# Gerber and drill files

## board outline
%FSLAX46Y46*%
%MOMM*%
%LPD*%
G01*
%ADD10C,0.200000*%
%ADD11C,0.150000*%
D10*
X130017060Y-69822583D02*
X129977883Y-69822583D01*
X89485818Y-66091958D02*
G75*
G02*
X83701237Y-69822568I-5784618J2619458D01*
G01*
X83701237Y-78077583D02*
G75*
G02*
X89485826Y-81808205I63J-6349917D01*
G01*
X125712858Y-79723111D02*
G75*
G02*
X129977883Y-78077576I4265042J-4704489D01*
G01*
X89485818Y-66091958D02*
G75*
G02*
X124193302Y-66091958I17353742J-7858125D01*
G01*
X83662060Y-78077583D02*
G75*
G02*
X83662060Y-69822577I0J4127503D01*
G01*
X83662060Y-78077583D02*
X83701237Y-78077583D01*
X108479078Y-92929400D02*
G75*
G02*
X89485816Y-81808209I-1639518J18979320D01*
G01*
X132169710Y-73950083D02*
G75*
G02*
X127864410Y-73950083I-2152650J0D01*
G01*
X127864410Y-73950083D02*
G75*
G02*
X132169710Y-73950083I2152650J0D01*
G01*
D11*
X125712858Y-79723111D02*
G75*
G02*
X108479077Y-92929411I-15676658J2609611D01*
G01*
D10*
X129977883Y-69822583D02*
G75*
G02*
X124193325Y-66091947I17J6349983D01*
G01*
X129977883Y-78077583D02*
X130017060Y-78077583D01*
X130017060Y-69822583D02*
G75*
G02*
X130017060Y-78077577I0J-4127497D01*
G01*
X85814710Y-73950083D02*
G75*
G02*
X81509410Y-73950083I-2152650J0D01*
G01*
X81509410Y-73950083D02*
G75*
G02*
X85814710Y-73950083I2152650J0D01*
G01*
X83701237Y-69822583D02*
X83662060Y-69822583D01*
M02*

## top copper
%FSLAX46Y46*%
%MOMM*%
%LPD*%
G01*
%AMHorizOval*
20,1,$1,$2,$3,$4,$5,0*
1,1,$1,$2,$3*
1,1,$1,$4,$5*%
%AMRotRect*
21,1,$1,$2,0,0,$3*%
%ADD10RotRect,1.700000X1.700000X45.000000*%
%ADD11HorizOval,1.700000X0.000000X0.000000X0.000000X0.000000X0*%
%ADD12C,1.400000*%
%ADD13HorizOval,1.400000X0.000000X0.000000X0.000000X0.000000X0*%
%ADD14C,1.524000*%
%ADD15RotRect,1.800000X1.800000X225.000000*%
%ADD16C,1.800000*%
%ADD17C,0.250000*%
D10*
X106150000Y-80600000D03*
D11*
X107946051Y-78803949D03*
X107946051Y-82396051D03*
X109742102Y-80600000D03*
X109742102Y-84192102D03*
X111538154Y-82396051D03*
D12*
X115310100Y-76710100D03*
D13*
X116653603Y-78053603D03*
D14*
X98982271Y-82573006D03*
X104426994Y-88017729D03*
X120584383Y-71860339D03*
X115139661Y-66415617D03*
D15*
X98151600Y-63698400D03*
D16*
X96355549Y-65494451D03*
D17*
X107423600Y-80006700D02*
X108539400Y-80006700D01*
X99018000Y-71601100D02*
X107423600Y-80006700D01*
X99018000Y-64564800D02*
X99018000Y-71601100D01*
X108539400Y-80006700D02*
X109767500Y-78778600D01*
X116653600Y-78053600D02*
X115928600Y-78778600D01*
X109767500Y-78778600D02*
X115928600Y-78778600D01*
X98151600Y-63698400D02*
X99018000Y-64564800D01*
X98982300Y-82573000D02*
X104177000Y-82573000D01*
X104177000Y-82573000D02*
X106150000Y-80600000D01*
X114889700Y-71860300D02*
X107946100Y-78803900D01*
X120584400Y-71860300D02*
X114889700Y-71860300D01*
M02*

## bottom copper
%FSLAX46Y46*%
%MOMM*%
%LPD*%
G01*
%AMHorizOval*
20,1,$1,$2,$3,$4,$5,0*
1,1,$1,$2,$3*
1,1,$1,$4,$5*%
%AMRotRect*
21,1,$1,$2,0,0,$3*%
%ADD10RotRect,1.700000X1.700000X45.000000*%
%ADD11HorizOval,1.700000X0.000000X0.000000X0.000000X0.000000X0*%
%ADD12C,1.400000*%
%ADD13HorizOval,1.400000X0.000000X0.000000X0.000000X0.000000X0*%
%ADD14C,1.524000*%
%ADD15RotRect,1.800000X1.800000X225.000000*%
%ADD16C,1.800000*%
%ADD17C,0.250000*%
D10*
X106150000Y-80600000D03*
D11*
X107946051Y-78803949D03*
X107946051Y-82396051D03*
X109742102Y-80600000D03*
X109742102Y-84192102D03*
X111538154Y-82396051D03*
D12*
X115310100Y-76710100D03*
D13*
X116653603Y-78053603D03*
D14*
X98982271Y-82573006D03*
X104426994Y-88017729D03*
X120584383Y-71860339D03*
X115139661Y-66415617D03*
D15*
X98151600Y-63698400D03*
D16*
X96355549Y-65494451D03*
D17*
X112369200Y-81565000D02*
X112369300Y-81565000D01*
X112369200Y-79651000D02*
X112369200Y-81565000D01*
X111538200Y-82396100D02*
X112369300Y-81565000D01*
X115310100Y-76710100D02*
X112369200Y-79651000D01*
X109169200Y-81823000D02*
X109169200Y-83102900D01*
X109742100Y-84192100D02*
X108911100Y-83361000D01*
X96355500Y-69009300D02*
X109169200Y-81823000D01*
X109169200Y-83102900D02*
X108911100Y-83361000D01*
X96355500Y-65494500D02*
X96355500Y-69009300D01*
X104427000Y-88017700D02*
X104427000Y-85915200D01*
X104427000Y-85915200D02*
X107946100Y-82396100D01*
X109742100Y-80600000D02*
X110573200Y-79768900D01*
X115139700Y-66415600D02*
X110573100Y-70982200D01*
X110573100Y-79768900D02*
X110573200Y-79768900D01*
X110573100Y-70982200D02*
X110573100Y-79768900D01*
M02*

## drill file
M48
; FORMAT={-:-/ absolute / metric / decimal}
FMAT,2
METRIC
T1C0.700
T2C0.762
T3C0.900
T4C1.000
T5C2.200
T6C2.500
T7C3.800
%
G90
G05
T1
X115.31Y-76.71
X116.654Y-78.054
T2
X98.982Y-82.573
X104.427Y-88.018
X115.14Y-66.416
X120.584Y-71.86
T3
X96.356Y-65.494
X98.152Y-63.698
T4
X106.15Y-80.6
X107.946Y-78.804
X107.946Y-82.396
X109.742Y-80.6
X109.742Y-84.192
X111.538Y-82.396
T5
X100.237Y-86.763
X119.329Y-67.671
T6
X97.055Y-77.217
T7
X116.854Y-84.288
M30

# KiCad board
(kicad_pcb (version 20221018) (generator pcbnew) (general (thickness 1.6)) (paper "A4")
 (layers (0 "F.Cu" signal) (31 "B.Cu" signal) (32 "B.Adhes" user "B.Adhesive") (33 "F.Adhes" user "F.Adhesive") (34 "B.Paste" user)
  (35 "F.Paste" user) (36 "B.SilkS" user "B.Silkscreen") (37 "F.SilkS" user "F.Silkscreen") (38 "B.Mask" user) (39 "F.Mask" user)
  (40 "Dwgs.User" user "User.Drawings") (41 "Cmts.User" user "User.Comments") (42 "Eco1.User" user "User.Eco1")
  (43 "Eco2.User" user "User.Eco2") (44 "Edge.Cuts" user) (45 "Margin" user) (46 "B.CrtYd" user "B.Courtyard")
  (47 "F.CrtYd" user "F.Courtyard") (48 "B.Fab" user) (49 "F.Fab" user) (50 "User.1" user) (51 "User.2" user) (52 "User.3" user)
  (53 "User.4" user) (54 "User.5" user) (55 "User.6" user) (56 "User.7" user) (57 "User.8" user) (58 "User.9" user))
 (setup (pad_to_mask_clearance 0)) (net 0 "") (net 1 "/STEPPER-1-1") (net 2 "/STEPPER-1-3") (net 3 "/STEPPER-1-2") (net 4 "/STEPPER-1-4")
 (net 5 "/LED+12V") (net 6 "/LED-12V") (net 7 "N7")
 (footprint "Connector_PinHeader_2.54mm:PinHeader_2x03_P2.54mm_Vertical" (layer "F.Cu") (at 106.15 80.6 45)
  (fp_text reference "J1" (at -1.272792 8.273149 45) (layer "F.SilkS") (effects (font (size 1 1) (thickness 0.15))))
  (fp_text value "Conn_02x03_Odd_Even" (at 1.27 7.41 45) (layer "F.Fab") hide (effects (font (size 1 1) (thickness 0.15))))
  (pad "1" thru_hole rect (at 0 0 45) (size 1.7 1.7) (drill 1) (layers "*.Cu" "*.Mask") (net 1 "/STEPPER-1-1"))
  (pad "2" thru_hole oval (at 2.54 0 45) (size 1.7 1.7) (drill 1) (layers "*.Cu" "*.Mask") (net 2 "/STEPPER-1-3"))
  (pad "3" thru_hole oval (at 0 2.54 45) (size 1.7 1.7) (drill 1) (layers "*.Cu" "*.Mask") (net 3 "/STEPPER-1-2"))
  (pad "4" thru_hole oval (at 2.54 2.54 45) (size 1.7 1.7) (drill 1) (layers "*.Cu" "*.Mask") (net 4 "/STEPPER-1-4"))
  (pad "5" thru_hole oval (at 0 5.08 45) (size 1.7 1.7) (drill 1) (layers "*.Cu" "*.Mask") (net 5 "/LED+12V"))
  (pad "6" thru_hole oval (at 2.54 5.08 45) (size 1.7 1.7) (drill 1) (layers "*.Cu" "*.Mask") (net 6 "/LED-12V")))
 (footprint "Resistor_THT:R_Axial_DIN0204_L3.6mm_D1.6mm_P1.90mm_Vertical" (layer "F.Cu") (at 115.3101 76.7101 -45)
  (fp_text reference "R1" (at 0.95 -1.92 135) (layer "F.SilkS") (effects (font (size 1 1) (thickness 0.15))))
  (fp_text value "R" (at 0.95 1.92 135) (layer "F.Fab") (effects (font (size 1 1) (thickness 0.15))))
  (pad "1" thru_hole circle (at 0 0 315) (size 1.4 1.4) (drill 0.7) (layers "*.Cu" "*.Mask") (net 6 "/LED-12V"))
  (pad "2" thru_hole oval (at 1.9 0 315) (size 1.4 1.4) (drill 0.7) (layers "*.Cu" "*.Mask") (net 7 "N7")))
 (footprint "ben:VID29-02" (layer "F.Cu") (at 109.9 77.1 45)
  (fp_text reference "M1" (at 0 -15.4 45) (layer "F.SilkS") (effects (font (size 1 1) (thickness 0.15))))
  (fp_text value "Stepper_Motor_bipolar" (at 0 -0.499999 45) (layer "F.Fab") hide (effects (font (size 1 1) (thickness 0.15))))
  (pad "" np_thru_hole circle (at -13.665 0 45) (size 2.2 2.2) (drill 2.2) (layers "*.Cu" "*.Mask"))
  (pad "" np_thru_hole circle (at -9.165 -9 45) (size 2.5 2.5) (drill 2.5) (layers "*.Cu" "*.Mask"))
  (pad "" np_thru_hole circle (at -0.165 10 45) (size 3.8 3.8) (drill 3.8) (layers "*.Cu" "*.Mask"))
  (pad "" np_thru_hole circle (at 13.335 0 45) (size 2.2 2.2) (drill 2.2) (layers "*.Cu" "*.Mask"))
  (pad "1" thru_hole circle (at -11.59 -3.85 45) (size 1.524 1.524) (drill 0.762) (layers "*.Cu" "*.Mask") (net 1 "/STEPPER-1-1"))
  (pad "2" thru_hole circle (at -11.59 3.85 45) (size 1.524 1.524) (drill 0.762) (layers "*.Cu" "*.Mask") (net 3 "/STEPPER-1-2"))
  (pad "3" thru_hole circle (at 11.26 3.85 45) (size 1.524 1.524) (drill 0.762) (layers "*.Cu" "*.Mask") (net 2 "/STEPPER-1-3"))
  (pad "4" thru_hole circle (at 11.26 -3.85 45) (size 1.524 1.524) (drill 0.762) (layers "*.Cu" "*.Mask") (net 4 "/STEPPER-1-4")))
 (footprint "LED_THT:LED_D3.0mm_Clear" (layer "B.Cu") (at 98.1516 63.6984 -135)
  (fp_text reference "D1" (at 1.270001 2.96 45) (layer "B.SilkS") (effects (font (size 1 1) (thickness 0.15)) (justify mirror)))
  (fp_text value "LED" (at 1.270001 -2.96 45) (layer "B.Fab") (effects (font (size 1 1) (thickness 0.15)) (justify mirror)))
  (pad "1" thru_hole rect (at 0 0 225) (size 1.8 1.8) (drill 0.9) (layers "*.Cu" "*.Mask") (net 7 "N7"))
  (pad "2" thru_hole circle (at 2.54 0 225) (size 1.8 1.8) (drill 0.9) (layers "*.Cu" "*.Mask") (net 5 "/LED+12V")))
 (gr_line (start 130.01706 69.822583) (end 129.977883 69.822583) (stroke (width 0.2) (type solid)) (layer "Edge.Cuts"))
 (gr_arc (start 89.485818 66.091958) (mid 87.142853 68.809031) (end 83.701237 69.822583) (stroke (width 0.2) (type solid))
  (layer "Edge.Cuts"))
 (gr_arc (start 83.701237 78.077583) (mid 87.142864 79.091118) (end 89.485818 81.808208) (stroke (width 0.2) (type solid))
  (layer "Edge.Cuts"))
 (gr_arc (start 125.712858 79.723111) (mid 127.692155 78.503231) (end 129.977883 78.077583) (stroke (width 0.2) (type solid))
  (layer "Edge.Cuts"))
 (gr_arc (start 89.485818 66.091958) (mid 106.83956 54.900083) (end 124.193302 66.091958) (stroke (width 0.2) (type solid))
  (layer "Edge.Cuts"))
 (gr_arc (start 83.66206 78.077583) (mid 79.53456 73.950083) (end 83.66206 69.822583) (stroke (width 0.2) (type solid)) (layer "Edge.Cuts"))
 (gr_line (start 83.66206 78.077583) (end 83.701237 78.077583) (stroke (width 0.2) (type solid)) (layer "Edge.Cuts"))
 (gr_arc (start 108.479078 92.9294) (mid 97.213843 90.389306) (end 89.485818 81.808208) (stroke (width 0.2) (type solid))
  (layer "Edge.Cuts"))
 (gr_circle (center 130.01706 73.950083) (end 127.86441 73.950083) (stroke (width 0.2) (type solid)) (fill none) (layer "Edge.Cuts"))
 (gr_arc (start 125.712858 79.723111) (mid 119.702734 89.728001) (end 108.479078 92.9294) (stroke (width 0.15) (type solid))
  (layer "Edge.Cuts"))
 (gr_arc (start 129.977883 69.822583) (mid 126.536265 68.809039) (end 124.193302 66.091958) (stroke (width 0.2) (type solid))
  (layer "Edge.Cuts"))
 (gr_line (start 129.977883 78.077583) (end 130.01706 78.077583) (stroke (width 0.2) (type solid)) (layer "Edge.Cuts"))
 (gr_arc (start 130.01706 69.822583) (mid 134.14456 73.950083) (end 130.01706 78.077583) (stroke (width 0.2) (type solid))
  (layer "Edge.Cuts"))
 (gr_circle (center 83.66206 73.950083) (end 81.50941 73.950083) (stroke (width 0.2) (type solid)) (fill none) (layer "Edge.Cuts"))
 (gr_line (start 83.701237 69.822583) (end 83.66206 69.822583) (stroke (width 0.2) (type solid)) (layer "Edge.Cuts"))
 (segment (start 107.4236 80.0067) (end 108.5394 80.0067) (width 0.25) (layer "F.Cu") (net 7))
 (segment (start 99.018 71.6011) (end 107.4236 80.0067) (width 0.25) (layer "F.Cu") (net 7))
 (segment (start 99.018 64.5648) (end 99.018 71.6011) (width 0.25) (layer "F.Cu") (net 7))
 (segment (start 108.5394 80.0067) (end 109.7675 78.7786) (width 0.25) (layer "F.Cu") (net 7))
 (segment (start 116.6536 78.0536) (end 115.9286 78.7786) (width 0.25) (layer "F.Cu") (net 7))
 (segment (start 109.7675 78.7786) (end 115.9286 78.7786) (width 0.25) (layer "F.Cu") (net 7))
 (segment (start 98.1516 63.6984) (end 99.018 64.5648) (width 0.25) (layer "F.Cu") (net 7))
 (segment (start 112.3692 81.565) (end 112.3693 81.565) (width 0.25) (layer "B.Cu") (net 6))
 (segment (start 112.3692 79.651) (end 112.3692 81.565) (width 0.25) (layer "B.Cu") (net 6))
 (segment (start 111.5382 82.3961) (end 112.3693 81.565) (width 0.25) (layer "B.Cu") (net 6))
 (segment (start 115.3101 76.7101) (end 112.3692 79.651) (width 0.25) (layer "B.Cu") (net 6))
 (segment (start 109.1692 81.823) (end 109.1692 83.1029) (width 0.25) (layer "B.Cu") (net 5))
 (segment (start 109.7421 84.1921) (end 108.9111 83.361) (width 0.25) (layer "B.Cu") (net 5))
 (segment (start 96.3555 69.0093) (end 109.1692 81.823) (width 0.25) (layer "B.Cu") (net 5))
 (segment (start 109.1692 83.1029) (end 108.9111 83.361) (width 0.25) (layer "B.Cu") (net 5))
 (segment (start 96.3555 65.4945) (end 96.3555 69.0093) (width 0.25) (layer "B.Cu") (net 5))
 (segment (start 98.9823 82.573) (end 104.177 82.573) (width 0.25) (layer "F.Cu") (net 1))
 (segment (start 104.177 82.573) (end 106.15 80.6) (width 0.25) (layer "F.Cu") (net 1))
 (segment (start 104.427 88.0177) (end 104.427 85.9152) (width 0.25) (layer "B.Cu") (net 3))
 (segment (start 104.427 85.9152) (end 107.9461 82.3961) (width 0.25) (layer "B.Cu") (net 3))
 (segment (start 114.8897 71.8603) (end 107.9461 78.8039) (width 0.25) (layer "F.Cu") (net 2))
 (segment (start 120.5844 71.8603) (end 114.8897 71.8603) (width 0.25) (layer "F.Cu") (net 2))
 (segment (start 109.7421 80.6) (end 110.5732 79.7689) (width 0.25) (layer "B.Cu") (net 4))
 (segment (start 115.1397 66.4156) (end 110.5731 70.9822) (width 0.25) (layer "B.Cu") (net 4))
 (segment (start 110.5731 79.7689) (end 110.5732 79.7689) (width 0.25) (layer "B.Cu") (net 4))
 (segment (start 110.5731 70.9822) (end 110.5731 79.7689) (width 0.25) (layer "B.Cu") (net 4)))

